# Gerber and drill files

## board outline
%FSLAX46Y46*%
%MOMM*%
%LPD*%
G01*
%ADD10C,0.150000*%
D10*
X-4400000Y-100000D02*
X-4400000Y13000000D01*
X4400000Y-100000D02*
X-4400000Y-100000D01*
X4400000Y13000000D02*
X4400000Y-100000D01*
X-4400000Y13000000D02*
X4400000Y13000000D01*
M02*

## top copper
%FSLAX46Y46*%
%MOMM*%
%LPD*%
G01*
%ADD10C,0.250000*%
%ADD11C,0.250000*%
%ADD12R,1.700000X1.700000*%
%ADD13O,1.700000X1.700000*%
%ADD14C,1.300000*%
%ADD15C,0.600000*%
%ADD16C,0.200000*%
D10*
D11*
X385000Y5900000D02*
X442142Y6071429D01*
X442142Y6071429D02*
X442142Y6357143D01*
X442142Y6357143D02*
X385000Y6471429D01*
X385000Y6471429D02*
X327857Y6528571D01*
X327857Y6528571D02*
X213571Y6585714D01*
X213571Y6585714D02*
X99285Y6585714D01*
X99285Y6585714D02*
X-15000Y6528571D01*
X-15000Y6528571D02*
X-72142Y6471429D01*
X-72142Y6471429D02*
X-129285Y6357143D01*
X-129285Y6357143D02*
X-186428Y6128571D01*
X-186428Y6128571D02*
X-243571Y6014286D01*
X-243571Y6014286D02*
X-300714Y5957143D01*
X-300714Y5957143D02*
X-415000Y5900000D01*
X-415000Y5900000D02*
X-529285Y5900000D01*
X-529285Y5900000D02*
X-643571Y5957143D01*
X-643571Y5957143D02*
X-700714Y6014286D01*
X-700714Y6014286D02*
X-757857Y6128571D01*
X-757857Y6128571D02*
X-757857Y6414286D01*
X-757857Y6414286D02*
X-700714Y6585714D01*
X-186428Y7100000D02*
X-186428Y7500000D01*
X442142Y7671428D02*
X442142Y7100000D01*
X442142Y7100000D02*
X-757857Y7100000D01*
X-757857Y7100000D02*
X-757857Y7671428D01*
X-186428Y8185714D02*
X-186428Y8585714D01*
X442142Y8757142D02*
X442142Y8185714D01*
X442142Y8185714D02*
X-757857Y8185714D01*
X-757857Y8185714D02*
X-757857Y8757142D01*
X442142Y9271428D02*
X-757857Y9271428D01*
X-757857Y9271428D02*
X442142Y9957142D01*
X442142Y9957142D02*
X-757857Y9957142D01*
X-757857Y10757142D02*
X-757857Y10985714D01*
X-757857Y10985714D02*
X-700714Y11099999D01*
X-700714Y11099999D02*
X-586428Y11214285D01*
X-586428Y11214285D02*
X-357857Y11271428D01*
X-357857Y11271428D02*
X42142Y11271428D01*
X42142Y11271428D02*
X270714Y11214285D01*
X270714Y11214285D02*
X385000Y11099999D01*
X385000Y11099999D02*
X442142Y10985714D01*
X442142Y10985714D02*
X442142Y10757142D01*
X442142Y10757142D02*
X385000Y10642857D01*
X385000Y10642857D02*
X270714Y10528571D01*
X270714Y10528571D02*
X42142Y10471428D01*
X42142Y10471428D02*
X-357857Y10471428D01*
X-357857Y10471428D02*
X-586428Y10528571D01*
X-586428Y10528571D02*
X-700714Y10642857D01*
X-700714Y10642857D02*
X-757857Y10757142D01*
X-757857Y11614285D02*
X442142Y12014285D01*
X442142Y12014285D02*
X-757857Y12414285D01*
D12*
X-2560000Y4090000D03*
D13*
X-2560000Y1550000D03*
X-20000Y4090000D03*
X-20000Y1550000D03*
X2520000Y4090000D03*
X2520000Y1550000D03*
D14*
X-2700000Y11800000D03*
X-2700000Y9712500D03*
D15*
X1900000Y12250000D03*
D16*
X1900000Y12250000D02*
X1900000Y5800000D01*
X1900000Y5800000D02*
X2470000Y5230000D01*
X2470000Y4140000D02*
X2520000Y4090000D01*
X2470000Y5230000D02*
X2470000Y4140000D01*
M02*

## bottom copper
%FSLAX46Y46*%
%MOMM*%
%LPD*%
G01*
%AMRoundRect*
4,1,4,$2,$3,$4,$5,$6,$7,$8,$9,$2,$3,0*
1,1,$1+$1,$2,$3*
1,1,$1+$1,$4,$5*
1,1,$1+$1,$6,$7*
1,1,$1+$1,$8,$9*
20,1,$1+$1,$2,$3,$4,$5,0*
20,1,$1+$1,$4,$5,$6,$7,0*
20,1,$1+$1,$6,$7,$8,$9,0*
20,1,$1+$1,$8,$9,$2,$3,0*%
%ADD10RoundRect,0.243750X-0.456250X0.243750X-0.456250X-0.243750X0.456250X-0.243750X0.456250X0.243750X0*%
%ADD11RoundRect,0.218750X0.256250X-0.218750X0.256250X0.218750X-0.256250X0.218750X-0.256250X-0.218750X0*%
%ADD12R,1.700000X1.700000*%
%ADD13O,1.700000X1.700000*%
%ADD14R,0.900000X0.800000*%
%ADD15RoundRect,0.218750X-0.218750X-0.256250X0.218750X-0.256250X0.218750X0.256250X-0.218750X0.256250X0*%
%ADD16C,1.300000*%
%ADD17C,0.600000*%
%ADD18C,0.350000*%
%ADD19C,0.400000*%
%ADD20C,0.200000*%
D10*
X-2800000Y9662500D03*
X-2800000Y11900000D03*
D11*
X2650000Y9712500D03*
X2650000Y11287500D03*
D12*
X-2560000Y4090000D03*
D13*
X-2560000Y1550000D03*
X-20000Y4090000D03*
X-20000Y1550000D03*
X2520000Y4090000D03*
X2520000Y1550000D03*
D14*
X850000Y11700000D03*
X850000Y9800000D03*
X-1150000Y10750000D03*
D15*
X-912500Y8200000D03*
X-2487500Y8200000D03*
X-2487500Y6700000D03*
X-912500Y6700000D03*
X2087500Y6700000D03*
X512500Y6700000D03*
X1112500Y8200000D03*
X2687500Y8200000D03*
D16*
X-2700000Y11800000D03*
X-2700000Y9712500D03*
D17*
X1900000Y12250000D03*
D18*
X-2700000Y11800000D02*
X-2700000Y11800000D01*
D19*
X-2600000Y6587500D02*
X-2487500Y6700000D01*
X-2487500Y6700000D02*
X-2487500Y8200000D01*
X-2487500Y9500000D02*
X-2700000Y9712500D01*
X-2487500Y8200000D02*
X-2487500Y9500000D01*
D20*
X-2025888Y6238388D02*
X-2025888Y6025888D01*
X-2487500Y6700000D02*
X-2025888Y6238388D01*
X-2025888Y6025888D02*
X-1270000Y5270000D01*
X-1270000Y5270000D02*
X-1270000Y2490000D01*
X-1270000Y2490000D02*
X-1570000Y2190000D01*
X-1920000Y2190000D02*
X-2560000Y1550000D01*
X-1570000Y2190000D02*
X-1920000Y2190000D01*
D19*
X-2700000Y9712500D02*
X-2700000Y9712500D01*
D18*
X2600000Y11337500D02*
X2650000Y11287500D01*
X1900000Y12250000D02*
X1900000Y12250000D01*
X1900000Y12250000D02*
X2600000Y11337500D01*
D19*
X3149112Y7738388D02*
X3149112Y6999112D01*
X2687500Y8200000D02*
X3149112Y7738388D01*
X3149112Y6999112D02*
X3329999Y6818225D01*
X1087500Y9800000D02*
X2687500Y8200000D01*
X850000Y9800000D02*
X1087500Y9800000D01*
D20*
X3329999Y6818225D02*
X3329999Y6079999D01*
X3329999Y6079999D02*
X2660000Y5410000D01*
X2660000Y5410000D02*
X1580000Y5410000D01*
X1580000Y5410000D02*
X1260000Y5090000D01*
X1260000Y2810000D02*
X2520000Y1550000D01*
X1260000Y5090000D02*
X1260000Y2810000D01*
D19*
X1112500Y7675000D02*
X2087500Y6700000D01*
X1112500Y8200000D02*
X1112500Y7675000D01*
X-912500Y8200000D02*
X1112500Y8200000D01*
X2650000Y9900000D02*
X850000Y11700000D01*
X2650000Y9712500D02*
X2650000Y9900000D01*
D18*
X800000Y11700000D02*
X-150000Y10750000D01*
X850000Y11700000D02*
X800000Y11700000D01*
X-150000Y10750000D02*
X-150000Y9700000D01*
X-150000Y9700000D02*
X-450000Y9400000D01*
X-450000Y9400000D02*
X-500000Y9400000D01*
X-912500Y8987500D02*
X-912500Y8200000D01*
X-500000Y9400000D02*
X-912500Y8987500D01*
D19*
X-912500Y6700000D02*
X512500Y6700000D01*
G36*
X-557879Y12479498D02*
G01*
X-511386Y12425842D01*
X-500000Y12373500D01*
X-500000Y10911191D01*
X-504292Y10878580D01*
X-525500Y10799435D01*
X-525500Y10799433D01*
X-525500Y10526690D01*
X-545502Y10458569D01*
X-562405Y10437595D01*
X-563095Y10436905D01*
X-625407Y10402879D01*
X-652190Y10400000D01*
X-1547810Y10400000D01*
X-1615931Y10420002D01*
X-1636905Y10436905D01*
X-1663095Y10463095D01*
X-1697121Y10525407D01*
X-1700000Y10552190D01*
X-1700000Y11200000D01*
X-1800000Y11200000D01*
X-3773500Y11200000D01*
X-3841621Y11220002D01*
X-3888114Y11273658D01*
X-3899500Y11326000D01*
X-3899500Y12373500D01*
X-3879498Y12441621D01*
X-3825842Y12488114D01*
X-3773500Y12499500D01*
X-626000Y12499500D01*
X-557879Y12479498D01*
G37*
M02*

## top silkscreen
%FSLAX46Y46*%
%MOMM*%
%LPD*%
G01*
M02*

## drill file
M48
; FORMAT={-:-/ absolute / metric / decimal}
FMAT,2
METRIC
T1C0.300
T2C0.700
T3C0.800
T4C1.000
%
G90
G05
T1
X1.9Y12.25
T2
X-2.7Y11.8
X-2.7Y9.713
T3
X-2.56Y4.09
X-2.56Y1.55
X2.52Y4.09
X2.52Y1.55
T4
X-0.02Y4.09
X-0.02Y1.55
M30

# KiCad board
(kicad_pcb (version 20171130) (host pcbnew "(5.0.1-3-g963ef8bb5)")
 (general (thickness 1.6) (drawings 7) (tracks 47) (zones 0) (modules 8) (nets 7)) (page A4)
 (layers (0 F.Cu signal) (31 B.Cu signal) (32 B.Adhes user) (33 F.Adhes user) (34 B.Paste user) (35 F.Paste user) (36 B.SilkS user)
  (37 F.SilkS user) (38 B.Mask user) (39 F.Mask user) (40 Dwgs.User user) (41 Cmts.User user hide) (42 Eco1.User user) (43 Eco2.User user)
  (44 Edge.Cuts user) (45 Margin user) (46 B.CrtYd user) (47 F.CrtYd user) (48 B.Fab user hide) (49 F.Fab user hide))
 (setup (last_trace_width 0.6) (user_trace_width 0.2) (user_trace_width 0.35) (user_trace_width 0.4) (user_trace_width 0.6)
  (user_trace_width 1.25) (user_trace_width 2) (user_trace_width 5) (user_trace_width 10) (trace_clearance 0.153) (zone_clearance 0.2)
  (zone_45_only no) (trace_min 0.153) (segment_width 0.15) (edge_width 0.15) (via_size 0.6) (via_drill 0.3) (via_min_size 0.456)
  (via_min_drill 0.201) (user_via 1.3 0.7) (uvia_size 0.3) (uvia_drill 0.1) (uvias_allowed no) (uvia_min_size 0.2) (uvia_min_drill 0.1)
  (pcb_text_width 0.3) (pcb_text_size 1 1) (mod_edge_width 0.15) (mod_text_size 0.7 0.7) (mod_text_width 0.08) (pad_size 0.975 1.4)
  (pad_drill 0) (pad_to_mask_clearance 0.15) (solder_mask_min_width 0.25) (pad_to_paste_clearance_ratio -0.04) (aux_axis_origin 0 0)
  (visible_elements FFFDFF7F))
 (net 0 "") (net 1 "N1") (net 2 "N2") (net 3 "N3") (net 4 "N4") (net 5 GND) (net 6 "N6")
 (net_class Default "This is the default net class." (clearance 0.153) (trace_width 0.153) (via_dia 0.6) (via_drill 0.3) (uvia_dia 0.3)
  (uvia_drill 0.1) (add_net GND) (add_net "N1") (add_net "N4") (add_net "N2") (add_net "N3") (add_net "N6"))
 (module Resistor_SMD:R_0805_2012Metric (layer B.Cu) (at -2.8 -10.6 270)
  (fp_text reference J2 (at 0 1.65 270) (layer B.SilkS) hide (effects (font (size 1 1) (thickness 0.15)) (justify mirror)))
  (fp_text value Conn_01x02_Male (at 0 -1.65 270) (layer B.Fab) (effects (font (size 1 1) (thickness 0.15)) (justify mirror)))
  (pad 2 smd roundrect (at 0.9375 0 270) (size 0.975 1.4) (layers B.Cu B.Paste B.Mask) (roundrect_rratio 0.25) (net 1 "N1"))
  (pad 1 smd roundrect (at -1.3 0 270) (size 0.975 1.4) (layers B.Cu B.Paste B.Mask) (roundrect_rratio 0.25) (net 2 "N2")))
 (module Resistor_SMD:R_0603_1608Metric (layer B.Cu) (at 2.65 -10.5 90)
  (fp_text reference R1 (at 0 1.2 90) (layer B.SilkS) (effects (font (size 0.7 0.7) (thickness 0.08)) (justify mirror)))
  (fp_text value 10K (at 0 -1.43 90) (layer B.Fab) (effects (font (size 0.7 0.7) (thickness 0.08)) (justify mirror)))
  (pad 1 smd roundrect (at -0.7875 0 90) (size 0.875 0.95) (layers B.Cu B.Paste B.Mask) (roundrect_rratio 0.25) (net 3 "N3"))
  (pad 2 smd roundrect (at 0.7875 0 90) (size 0.875 0.95) (layers B.Cu B.Paste B.Mask) (roundrect_rratio 0.25) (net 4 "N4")))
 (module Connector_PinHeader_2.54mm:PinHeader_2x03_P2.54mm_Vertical (layer B.Cu) (at -2.56 -4.09 270)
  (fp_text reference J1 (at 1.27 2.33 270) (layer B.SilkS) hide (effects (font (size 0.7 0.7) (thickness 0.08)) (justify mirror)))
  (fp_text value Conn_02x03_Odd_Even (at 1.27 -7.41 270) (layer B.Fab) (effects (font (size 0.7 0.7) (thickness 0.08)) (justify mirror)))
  (pad 1 thru_hole rect (at 0 0 270) (size 1.7 1.7) (drill 0.8) (layers *.Cu *.Mask))
  (pad 2 thru_hole oval (at 2.54 0 270) (size 1.7 1.7) (drill 0.8) (layers *.Cu *.Mask) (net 1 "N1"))
  (pad 3 thru_hole oval (at 0 -2.54 270) (size 1.7 1.7) (drill 1) (layers *.Cu *.Mask))
  (pad 4 thru_hole oval (at 2.54 -2.54 270) (size 1.7 1.7) (drill 1) (layers *.Cu *.Mask))
  (pad 5 thru_hole oval (at 0 -5.08 270) (size 1.7 1.7) (drill 0.8) (layers *.Cu *.Mask) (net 4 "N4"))
  (pad 6 thru_hole oval (at 2.54 -5.08 270) (size 1.7 1.7) (drill 0.8) (layers *.Cu *.Mask) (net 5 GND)))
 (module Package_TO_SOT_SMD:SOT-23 (layer B.Cu) (at -0.15 -10.75 180)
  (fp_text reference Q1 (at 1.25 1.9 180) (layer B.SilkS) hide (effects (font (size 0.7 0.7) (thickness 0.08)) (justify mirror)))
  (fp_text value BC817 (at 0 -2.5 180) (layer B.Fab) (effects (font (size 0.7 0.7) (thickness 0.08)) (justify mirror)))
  (pad 1 smd rect (at -1 0.95 180) (size 0.9 0.8) (layers B.Cu B.Paste B.Mask) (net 3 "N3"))
  (pad 2 smd rect (at -1 -0.95 180) (size 0.9 0.8) (layers B.Cu B.Paste B.Mask) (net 5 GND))
  (pad 3 smd rect (at 1 0 180) (size 0.9 0.8) (layers B.Cu B.Paste B.Mask) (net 2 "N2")))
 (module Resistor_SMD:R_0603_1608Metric (layer B.Cu) (at -1.7 -8.2)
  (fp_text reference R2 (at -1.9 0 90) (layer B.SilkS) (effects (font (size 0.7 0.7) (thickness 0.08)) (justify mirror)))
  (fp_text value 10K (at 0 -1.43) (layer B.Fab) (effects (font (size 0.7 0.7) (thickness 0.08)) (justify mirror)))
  (pad 2 smd roundrect (at 0.7875 0) (size 0.875 0.95) (layers B.Cu B.Paste B.Mask) (roundrect_rratio 0.25) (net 3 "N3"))
  (pad 1 smd roundrect (at -0.7875 0) (size 0.875 0.95) (layers B.Cu B.Paste B.Mask) (roundrect_rratio 0.25) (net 1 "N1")))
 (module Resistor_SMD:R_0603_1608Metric (layer B.Cu) (at -1.7 -6.7)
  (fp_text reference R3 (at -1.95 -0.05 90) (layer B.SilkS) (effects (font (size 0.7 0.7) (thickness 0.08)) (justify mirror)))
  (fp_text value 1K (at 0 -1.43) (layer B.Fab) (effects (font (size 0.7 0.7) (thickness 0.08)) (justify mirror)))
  (pad 1 smd roundrect (at -0.7875 0) (size 0.875 0.95) (layers B.Cu B.Paste B.Mask) (roundrect_rratio 0.25) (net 1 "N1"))
  (pad 2 smd roundrect (at 0.7875 0) (size 0.875 0.95) (layers B.Cu B.Paste B.Mask) (roundrect_rratio 0.25) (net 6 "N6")))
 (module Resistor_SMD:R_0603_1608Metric (layer B.Cu) (at 1.3 -6.7)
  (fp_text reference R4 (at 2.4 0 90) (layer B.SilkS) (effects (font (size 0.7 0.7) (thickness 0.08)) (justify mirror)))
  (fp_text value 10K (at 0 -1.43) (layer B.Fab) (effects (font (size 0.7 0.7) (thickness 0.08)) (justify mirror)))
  (pad 2 smd roundrect (at 0.7875 0) (size 0.875 0.95) (layers B.Cu B.Paste B.Mask) (roundrect_rratio 0.25) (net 3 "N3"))
  (pad 1 smd roundrect (at -0.7875 0) (size 0.875 0.95) (layers B.Cu B.Paste B.Mask) (roundrect_rratio 0.25) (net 6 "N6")))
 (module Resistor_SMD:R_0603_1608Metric (layer B.Cu) (at 1.9 -8.2)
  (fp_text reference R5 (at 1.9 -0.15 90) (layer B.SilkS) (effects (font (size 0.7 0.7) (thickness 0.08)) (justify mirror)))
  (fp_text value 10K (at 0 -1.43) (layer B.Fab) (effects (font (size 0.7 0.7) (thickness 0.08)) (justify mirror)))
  (pad 1 smd roundrect (at -0.7875 0) (size 0.875 0.95) (layers B.Cu B.Paste B.Mask) (roundrect_rratio 0.25) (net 3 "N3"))
  (pad 2 smd roundrect (at 0.7875 0) (size 0.875 0.95) (layers B.Cu B.Paste B.Mask) (roundrect_rratio 0.25) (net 5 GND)))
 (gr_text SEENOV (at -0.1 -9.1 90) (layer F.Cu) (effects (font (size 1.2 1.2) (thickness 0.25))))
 (gr_line (start -4.4 0.1) (end -4.4 -13) (layer Edge.Cuts) (width 0.15))
 (gr_line (start 4.4 0.1) (end -4.4 0.1) (layer Edge.Cuts) (width 0.15))
 (gr_line (start 4.4 -13) (end 4.4 0.1) (layer Edge.Cuts) (width 0.15))
 (gr_line (start -4.4 -13) (end 4.4 -13) (layer Edge.Cuts) (width 0.15))
 (segment (start -2.7 -11.8) (end -2.7 -11.8) (width 0.35) (layer B.Cu) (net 2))
 (via (at -2.7 -11.8) (size 1.3) (drill 0.7) (layers F.Cu B.Cu) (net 2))
 (segment (start -2.6 -6.5875) (end -2.4875 -6.7) (width 0.4) (layer B.Cu) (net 1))
 (segment (start -2.4875 -6.7) (end -2.4875 -8.2) (width 0.4) (layer B.Cu) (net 1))
 (segment (start -2.4875 -9.5) (end -2.7 -9.7125) (width 0.4) (layer B.Cu) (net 1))
 (segment (start -2.4875 -8.2) (end -2.4875 -9.5) (width 0.4) (layer B.Cu) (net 1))
 (segment (start -2.025888 -6.238388) (end -2.025888 -6.025888) (width 0.2) (layer B.Cu) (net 1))
 (segment (start -2.4875 -6.7) (end -2.025888 -6.238388) (width 0.2) (layer B.Cu) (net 1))
 (segment (start -2.025888 -6.025888) (end -1.27 -5.27) (width 0.2) (layer B.Cu) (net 1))
 (segment (start -1.27 -5.27) (end -1.27 -2.49) (width 0.2) (layer B.Cu) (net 1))
 (segment (start -1.27 -2.49) (end -1.57 -2.19) (width 0.2) (layer B.Cu) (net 1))
 (segment (start -1.92 -2.19) (end -2.56 -1.55) (width 0.2) (layer B.Cu) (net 1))
 (segment (start -1.57 -2.19) (end -1.92 -2.19) (width 0.2) (layer B.Cu) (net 1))
 (segment (start -2.7 -9.7125) (end -2.7 -9.7125) (width 0.4) (layer B.Cu) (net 1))
 (via (at -2.7 -9.7125) (size 1.3) (drill 0.7) (layers F.Cu B.Cu) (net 1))
 (segment (start 2.6 -11.3375) (end 2.65 -11.2875) (width 0.35) (layer B.Cu) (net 4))
 (segment (start 1.9 -12.25) (end 1.9 -12.25) (width 0.35) (layer B.Cu) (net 4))
 (segment (start 1.9 -12.25) (end 2.6 -11.3375) (width 0.35) (layer B.Cu) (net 4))
 (via (at 1.9 -12.25) (size 0.6) (drill 0.3) (layers F.Cu B.Cu) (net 4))
 (segment (start 1.9 -12.25) (end 1.9 -5.8) (width 0.2) (layer F.Cu) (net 4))
 (segment (start 1.9 -5.8) (end 2.47 -5.23) (width 0.2) (layer F.Cu) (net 4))
 (segment (start 2.47 -4.14) (end 2.52 -4.09) (width 0.2) (layer F.Cu) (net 4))
 (segment (start 2.47 -5.23) (end 2.47 -4.14) (width 0.2) (layer F.Cu) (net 4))
 (segment (start 3.149112 -7.738388) (end 3.149112 -6.999112) (width 0.4) (layer B.Cu) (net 5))
 (segment (start 2.6875 -8.2) (end 3.149112 -7.738388) (width 0.4) (layer B.Cu) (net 5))
 (segment (start 3.149112 -6.999112) (end 3.329999 -6.818225) (width 0.4) (layer B.Cu) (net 5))
 (segment (start 1.0875 -9.8) (end 2.6875 -8.2) (width 0.4) (layer B.Cu) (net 5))
 (segment (start 0.85 -9.8) (end 1.0875 -9.8) (width 0.4) (layer B.Cu) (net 5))
 (segment (start 3.329999 -6.818225) (end 3.329999 -6.079999) (width 0.2) (layer B.Cu) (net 5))
 (segment (start 3.329999 -6.079999) (end 2.66 -5.41) (width 0.2) (layer B.Cu) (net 5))
 (segment (start 2.66 -5.41) (end 1.58 -5.41) (width 0.2) (layer B.Cu) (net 5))
 (segment (start 1.58 -5.41) (end 1.26 -5.09) (width 0.2) (layer B.Cu) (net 5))
 (segment (start 1.26 -2.81) (end 2.52 -1.55) (width 0.2) (layer B.Cu) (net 5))
 (segment (start 1.26 -5.09) (end 1.26 -2.81) (width 0.2) (layer B.Cu) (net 5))
 (segment (start 1.1125 -7.675) (end 2.0875 -6.7) (width 0.4) (layer B.Cu) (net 3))
 (segment (start 1.1125 -8.2) (end 1.1125 -7.675) (width 0.4) (layer B.Cu) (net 3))
 (segment (start -0.9125 -8.2) (end 1.1125 -8.2) (width 0.4) (layer B.Cu) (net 3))
 (segment (start 2.65 -9.9) (end 0.85 -11.7) (width 0.4) (layer B.Cu) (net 3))
 (segment (start 2.65 -9.7125) (end 2.65 -9.9) (width 0.4) (layer B.Cu) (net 3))
 (segment (start 0.8 -11.7) (end -0.15 -10.75) (width 0.35) (layer B.Cu) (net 3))
 (segment (start 0.85 -11.7) (end 0.8 -11.7) (width 0.35) (layer B.Cu) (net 3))
 (segment (start -0.15 -10.75) (end -0.15 -9.7) (width 0.35) (layer B.Cu) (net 3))
 (segment (start -0.15 -9.7) (end -0.45 -9.4) (width 0.35) (layer B.Cu) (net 3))
 (segment (start -0.45 -9.4) (end -0.5 -9.4) (width 0.35) (layer B.Cu) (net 3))
 (segment (start -0.9125 -8.9875) (end -0.9125 -8.2) (width 0.35) (layer B.Cu) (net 3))
 (segment (start -0.5 -9.4) (end -0.9125 -8.9875) (width 0.35) (layer B.Cu) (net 3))
 (segment (start -0.9125 -6.7) (end 0.5125 -6.7) (width 0.4) (layer B.Cu) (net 6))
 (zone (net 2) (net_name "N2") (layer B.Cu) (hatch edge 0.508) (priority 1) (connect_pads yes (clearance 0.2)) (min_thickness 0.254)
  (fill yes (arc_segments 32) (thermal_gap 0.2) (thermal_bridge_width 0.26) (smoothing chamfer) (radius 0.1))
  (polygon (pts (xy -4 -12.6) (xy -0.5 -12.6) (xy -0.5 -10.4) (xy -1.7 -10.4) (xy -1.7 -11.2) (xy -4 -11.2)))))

